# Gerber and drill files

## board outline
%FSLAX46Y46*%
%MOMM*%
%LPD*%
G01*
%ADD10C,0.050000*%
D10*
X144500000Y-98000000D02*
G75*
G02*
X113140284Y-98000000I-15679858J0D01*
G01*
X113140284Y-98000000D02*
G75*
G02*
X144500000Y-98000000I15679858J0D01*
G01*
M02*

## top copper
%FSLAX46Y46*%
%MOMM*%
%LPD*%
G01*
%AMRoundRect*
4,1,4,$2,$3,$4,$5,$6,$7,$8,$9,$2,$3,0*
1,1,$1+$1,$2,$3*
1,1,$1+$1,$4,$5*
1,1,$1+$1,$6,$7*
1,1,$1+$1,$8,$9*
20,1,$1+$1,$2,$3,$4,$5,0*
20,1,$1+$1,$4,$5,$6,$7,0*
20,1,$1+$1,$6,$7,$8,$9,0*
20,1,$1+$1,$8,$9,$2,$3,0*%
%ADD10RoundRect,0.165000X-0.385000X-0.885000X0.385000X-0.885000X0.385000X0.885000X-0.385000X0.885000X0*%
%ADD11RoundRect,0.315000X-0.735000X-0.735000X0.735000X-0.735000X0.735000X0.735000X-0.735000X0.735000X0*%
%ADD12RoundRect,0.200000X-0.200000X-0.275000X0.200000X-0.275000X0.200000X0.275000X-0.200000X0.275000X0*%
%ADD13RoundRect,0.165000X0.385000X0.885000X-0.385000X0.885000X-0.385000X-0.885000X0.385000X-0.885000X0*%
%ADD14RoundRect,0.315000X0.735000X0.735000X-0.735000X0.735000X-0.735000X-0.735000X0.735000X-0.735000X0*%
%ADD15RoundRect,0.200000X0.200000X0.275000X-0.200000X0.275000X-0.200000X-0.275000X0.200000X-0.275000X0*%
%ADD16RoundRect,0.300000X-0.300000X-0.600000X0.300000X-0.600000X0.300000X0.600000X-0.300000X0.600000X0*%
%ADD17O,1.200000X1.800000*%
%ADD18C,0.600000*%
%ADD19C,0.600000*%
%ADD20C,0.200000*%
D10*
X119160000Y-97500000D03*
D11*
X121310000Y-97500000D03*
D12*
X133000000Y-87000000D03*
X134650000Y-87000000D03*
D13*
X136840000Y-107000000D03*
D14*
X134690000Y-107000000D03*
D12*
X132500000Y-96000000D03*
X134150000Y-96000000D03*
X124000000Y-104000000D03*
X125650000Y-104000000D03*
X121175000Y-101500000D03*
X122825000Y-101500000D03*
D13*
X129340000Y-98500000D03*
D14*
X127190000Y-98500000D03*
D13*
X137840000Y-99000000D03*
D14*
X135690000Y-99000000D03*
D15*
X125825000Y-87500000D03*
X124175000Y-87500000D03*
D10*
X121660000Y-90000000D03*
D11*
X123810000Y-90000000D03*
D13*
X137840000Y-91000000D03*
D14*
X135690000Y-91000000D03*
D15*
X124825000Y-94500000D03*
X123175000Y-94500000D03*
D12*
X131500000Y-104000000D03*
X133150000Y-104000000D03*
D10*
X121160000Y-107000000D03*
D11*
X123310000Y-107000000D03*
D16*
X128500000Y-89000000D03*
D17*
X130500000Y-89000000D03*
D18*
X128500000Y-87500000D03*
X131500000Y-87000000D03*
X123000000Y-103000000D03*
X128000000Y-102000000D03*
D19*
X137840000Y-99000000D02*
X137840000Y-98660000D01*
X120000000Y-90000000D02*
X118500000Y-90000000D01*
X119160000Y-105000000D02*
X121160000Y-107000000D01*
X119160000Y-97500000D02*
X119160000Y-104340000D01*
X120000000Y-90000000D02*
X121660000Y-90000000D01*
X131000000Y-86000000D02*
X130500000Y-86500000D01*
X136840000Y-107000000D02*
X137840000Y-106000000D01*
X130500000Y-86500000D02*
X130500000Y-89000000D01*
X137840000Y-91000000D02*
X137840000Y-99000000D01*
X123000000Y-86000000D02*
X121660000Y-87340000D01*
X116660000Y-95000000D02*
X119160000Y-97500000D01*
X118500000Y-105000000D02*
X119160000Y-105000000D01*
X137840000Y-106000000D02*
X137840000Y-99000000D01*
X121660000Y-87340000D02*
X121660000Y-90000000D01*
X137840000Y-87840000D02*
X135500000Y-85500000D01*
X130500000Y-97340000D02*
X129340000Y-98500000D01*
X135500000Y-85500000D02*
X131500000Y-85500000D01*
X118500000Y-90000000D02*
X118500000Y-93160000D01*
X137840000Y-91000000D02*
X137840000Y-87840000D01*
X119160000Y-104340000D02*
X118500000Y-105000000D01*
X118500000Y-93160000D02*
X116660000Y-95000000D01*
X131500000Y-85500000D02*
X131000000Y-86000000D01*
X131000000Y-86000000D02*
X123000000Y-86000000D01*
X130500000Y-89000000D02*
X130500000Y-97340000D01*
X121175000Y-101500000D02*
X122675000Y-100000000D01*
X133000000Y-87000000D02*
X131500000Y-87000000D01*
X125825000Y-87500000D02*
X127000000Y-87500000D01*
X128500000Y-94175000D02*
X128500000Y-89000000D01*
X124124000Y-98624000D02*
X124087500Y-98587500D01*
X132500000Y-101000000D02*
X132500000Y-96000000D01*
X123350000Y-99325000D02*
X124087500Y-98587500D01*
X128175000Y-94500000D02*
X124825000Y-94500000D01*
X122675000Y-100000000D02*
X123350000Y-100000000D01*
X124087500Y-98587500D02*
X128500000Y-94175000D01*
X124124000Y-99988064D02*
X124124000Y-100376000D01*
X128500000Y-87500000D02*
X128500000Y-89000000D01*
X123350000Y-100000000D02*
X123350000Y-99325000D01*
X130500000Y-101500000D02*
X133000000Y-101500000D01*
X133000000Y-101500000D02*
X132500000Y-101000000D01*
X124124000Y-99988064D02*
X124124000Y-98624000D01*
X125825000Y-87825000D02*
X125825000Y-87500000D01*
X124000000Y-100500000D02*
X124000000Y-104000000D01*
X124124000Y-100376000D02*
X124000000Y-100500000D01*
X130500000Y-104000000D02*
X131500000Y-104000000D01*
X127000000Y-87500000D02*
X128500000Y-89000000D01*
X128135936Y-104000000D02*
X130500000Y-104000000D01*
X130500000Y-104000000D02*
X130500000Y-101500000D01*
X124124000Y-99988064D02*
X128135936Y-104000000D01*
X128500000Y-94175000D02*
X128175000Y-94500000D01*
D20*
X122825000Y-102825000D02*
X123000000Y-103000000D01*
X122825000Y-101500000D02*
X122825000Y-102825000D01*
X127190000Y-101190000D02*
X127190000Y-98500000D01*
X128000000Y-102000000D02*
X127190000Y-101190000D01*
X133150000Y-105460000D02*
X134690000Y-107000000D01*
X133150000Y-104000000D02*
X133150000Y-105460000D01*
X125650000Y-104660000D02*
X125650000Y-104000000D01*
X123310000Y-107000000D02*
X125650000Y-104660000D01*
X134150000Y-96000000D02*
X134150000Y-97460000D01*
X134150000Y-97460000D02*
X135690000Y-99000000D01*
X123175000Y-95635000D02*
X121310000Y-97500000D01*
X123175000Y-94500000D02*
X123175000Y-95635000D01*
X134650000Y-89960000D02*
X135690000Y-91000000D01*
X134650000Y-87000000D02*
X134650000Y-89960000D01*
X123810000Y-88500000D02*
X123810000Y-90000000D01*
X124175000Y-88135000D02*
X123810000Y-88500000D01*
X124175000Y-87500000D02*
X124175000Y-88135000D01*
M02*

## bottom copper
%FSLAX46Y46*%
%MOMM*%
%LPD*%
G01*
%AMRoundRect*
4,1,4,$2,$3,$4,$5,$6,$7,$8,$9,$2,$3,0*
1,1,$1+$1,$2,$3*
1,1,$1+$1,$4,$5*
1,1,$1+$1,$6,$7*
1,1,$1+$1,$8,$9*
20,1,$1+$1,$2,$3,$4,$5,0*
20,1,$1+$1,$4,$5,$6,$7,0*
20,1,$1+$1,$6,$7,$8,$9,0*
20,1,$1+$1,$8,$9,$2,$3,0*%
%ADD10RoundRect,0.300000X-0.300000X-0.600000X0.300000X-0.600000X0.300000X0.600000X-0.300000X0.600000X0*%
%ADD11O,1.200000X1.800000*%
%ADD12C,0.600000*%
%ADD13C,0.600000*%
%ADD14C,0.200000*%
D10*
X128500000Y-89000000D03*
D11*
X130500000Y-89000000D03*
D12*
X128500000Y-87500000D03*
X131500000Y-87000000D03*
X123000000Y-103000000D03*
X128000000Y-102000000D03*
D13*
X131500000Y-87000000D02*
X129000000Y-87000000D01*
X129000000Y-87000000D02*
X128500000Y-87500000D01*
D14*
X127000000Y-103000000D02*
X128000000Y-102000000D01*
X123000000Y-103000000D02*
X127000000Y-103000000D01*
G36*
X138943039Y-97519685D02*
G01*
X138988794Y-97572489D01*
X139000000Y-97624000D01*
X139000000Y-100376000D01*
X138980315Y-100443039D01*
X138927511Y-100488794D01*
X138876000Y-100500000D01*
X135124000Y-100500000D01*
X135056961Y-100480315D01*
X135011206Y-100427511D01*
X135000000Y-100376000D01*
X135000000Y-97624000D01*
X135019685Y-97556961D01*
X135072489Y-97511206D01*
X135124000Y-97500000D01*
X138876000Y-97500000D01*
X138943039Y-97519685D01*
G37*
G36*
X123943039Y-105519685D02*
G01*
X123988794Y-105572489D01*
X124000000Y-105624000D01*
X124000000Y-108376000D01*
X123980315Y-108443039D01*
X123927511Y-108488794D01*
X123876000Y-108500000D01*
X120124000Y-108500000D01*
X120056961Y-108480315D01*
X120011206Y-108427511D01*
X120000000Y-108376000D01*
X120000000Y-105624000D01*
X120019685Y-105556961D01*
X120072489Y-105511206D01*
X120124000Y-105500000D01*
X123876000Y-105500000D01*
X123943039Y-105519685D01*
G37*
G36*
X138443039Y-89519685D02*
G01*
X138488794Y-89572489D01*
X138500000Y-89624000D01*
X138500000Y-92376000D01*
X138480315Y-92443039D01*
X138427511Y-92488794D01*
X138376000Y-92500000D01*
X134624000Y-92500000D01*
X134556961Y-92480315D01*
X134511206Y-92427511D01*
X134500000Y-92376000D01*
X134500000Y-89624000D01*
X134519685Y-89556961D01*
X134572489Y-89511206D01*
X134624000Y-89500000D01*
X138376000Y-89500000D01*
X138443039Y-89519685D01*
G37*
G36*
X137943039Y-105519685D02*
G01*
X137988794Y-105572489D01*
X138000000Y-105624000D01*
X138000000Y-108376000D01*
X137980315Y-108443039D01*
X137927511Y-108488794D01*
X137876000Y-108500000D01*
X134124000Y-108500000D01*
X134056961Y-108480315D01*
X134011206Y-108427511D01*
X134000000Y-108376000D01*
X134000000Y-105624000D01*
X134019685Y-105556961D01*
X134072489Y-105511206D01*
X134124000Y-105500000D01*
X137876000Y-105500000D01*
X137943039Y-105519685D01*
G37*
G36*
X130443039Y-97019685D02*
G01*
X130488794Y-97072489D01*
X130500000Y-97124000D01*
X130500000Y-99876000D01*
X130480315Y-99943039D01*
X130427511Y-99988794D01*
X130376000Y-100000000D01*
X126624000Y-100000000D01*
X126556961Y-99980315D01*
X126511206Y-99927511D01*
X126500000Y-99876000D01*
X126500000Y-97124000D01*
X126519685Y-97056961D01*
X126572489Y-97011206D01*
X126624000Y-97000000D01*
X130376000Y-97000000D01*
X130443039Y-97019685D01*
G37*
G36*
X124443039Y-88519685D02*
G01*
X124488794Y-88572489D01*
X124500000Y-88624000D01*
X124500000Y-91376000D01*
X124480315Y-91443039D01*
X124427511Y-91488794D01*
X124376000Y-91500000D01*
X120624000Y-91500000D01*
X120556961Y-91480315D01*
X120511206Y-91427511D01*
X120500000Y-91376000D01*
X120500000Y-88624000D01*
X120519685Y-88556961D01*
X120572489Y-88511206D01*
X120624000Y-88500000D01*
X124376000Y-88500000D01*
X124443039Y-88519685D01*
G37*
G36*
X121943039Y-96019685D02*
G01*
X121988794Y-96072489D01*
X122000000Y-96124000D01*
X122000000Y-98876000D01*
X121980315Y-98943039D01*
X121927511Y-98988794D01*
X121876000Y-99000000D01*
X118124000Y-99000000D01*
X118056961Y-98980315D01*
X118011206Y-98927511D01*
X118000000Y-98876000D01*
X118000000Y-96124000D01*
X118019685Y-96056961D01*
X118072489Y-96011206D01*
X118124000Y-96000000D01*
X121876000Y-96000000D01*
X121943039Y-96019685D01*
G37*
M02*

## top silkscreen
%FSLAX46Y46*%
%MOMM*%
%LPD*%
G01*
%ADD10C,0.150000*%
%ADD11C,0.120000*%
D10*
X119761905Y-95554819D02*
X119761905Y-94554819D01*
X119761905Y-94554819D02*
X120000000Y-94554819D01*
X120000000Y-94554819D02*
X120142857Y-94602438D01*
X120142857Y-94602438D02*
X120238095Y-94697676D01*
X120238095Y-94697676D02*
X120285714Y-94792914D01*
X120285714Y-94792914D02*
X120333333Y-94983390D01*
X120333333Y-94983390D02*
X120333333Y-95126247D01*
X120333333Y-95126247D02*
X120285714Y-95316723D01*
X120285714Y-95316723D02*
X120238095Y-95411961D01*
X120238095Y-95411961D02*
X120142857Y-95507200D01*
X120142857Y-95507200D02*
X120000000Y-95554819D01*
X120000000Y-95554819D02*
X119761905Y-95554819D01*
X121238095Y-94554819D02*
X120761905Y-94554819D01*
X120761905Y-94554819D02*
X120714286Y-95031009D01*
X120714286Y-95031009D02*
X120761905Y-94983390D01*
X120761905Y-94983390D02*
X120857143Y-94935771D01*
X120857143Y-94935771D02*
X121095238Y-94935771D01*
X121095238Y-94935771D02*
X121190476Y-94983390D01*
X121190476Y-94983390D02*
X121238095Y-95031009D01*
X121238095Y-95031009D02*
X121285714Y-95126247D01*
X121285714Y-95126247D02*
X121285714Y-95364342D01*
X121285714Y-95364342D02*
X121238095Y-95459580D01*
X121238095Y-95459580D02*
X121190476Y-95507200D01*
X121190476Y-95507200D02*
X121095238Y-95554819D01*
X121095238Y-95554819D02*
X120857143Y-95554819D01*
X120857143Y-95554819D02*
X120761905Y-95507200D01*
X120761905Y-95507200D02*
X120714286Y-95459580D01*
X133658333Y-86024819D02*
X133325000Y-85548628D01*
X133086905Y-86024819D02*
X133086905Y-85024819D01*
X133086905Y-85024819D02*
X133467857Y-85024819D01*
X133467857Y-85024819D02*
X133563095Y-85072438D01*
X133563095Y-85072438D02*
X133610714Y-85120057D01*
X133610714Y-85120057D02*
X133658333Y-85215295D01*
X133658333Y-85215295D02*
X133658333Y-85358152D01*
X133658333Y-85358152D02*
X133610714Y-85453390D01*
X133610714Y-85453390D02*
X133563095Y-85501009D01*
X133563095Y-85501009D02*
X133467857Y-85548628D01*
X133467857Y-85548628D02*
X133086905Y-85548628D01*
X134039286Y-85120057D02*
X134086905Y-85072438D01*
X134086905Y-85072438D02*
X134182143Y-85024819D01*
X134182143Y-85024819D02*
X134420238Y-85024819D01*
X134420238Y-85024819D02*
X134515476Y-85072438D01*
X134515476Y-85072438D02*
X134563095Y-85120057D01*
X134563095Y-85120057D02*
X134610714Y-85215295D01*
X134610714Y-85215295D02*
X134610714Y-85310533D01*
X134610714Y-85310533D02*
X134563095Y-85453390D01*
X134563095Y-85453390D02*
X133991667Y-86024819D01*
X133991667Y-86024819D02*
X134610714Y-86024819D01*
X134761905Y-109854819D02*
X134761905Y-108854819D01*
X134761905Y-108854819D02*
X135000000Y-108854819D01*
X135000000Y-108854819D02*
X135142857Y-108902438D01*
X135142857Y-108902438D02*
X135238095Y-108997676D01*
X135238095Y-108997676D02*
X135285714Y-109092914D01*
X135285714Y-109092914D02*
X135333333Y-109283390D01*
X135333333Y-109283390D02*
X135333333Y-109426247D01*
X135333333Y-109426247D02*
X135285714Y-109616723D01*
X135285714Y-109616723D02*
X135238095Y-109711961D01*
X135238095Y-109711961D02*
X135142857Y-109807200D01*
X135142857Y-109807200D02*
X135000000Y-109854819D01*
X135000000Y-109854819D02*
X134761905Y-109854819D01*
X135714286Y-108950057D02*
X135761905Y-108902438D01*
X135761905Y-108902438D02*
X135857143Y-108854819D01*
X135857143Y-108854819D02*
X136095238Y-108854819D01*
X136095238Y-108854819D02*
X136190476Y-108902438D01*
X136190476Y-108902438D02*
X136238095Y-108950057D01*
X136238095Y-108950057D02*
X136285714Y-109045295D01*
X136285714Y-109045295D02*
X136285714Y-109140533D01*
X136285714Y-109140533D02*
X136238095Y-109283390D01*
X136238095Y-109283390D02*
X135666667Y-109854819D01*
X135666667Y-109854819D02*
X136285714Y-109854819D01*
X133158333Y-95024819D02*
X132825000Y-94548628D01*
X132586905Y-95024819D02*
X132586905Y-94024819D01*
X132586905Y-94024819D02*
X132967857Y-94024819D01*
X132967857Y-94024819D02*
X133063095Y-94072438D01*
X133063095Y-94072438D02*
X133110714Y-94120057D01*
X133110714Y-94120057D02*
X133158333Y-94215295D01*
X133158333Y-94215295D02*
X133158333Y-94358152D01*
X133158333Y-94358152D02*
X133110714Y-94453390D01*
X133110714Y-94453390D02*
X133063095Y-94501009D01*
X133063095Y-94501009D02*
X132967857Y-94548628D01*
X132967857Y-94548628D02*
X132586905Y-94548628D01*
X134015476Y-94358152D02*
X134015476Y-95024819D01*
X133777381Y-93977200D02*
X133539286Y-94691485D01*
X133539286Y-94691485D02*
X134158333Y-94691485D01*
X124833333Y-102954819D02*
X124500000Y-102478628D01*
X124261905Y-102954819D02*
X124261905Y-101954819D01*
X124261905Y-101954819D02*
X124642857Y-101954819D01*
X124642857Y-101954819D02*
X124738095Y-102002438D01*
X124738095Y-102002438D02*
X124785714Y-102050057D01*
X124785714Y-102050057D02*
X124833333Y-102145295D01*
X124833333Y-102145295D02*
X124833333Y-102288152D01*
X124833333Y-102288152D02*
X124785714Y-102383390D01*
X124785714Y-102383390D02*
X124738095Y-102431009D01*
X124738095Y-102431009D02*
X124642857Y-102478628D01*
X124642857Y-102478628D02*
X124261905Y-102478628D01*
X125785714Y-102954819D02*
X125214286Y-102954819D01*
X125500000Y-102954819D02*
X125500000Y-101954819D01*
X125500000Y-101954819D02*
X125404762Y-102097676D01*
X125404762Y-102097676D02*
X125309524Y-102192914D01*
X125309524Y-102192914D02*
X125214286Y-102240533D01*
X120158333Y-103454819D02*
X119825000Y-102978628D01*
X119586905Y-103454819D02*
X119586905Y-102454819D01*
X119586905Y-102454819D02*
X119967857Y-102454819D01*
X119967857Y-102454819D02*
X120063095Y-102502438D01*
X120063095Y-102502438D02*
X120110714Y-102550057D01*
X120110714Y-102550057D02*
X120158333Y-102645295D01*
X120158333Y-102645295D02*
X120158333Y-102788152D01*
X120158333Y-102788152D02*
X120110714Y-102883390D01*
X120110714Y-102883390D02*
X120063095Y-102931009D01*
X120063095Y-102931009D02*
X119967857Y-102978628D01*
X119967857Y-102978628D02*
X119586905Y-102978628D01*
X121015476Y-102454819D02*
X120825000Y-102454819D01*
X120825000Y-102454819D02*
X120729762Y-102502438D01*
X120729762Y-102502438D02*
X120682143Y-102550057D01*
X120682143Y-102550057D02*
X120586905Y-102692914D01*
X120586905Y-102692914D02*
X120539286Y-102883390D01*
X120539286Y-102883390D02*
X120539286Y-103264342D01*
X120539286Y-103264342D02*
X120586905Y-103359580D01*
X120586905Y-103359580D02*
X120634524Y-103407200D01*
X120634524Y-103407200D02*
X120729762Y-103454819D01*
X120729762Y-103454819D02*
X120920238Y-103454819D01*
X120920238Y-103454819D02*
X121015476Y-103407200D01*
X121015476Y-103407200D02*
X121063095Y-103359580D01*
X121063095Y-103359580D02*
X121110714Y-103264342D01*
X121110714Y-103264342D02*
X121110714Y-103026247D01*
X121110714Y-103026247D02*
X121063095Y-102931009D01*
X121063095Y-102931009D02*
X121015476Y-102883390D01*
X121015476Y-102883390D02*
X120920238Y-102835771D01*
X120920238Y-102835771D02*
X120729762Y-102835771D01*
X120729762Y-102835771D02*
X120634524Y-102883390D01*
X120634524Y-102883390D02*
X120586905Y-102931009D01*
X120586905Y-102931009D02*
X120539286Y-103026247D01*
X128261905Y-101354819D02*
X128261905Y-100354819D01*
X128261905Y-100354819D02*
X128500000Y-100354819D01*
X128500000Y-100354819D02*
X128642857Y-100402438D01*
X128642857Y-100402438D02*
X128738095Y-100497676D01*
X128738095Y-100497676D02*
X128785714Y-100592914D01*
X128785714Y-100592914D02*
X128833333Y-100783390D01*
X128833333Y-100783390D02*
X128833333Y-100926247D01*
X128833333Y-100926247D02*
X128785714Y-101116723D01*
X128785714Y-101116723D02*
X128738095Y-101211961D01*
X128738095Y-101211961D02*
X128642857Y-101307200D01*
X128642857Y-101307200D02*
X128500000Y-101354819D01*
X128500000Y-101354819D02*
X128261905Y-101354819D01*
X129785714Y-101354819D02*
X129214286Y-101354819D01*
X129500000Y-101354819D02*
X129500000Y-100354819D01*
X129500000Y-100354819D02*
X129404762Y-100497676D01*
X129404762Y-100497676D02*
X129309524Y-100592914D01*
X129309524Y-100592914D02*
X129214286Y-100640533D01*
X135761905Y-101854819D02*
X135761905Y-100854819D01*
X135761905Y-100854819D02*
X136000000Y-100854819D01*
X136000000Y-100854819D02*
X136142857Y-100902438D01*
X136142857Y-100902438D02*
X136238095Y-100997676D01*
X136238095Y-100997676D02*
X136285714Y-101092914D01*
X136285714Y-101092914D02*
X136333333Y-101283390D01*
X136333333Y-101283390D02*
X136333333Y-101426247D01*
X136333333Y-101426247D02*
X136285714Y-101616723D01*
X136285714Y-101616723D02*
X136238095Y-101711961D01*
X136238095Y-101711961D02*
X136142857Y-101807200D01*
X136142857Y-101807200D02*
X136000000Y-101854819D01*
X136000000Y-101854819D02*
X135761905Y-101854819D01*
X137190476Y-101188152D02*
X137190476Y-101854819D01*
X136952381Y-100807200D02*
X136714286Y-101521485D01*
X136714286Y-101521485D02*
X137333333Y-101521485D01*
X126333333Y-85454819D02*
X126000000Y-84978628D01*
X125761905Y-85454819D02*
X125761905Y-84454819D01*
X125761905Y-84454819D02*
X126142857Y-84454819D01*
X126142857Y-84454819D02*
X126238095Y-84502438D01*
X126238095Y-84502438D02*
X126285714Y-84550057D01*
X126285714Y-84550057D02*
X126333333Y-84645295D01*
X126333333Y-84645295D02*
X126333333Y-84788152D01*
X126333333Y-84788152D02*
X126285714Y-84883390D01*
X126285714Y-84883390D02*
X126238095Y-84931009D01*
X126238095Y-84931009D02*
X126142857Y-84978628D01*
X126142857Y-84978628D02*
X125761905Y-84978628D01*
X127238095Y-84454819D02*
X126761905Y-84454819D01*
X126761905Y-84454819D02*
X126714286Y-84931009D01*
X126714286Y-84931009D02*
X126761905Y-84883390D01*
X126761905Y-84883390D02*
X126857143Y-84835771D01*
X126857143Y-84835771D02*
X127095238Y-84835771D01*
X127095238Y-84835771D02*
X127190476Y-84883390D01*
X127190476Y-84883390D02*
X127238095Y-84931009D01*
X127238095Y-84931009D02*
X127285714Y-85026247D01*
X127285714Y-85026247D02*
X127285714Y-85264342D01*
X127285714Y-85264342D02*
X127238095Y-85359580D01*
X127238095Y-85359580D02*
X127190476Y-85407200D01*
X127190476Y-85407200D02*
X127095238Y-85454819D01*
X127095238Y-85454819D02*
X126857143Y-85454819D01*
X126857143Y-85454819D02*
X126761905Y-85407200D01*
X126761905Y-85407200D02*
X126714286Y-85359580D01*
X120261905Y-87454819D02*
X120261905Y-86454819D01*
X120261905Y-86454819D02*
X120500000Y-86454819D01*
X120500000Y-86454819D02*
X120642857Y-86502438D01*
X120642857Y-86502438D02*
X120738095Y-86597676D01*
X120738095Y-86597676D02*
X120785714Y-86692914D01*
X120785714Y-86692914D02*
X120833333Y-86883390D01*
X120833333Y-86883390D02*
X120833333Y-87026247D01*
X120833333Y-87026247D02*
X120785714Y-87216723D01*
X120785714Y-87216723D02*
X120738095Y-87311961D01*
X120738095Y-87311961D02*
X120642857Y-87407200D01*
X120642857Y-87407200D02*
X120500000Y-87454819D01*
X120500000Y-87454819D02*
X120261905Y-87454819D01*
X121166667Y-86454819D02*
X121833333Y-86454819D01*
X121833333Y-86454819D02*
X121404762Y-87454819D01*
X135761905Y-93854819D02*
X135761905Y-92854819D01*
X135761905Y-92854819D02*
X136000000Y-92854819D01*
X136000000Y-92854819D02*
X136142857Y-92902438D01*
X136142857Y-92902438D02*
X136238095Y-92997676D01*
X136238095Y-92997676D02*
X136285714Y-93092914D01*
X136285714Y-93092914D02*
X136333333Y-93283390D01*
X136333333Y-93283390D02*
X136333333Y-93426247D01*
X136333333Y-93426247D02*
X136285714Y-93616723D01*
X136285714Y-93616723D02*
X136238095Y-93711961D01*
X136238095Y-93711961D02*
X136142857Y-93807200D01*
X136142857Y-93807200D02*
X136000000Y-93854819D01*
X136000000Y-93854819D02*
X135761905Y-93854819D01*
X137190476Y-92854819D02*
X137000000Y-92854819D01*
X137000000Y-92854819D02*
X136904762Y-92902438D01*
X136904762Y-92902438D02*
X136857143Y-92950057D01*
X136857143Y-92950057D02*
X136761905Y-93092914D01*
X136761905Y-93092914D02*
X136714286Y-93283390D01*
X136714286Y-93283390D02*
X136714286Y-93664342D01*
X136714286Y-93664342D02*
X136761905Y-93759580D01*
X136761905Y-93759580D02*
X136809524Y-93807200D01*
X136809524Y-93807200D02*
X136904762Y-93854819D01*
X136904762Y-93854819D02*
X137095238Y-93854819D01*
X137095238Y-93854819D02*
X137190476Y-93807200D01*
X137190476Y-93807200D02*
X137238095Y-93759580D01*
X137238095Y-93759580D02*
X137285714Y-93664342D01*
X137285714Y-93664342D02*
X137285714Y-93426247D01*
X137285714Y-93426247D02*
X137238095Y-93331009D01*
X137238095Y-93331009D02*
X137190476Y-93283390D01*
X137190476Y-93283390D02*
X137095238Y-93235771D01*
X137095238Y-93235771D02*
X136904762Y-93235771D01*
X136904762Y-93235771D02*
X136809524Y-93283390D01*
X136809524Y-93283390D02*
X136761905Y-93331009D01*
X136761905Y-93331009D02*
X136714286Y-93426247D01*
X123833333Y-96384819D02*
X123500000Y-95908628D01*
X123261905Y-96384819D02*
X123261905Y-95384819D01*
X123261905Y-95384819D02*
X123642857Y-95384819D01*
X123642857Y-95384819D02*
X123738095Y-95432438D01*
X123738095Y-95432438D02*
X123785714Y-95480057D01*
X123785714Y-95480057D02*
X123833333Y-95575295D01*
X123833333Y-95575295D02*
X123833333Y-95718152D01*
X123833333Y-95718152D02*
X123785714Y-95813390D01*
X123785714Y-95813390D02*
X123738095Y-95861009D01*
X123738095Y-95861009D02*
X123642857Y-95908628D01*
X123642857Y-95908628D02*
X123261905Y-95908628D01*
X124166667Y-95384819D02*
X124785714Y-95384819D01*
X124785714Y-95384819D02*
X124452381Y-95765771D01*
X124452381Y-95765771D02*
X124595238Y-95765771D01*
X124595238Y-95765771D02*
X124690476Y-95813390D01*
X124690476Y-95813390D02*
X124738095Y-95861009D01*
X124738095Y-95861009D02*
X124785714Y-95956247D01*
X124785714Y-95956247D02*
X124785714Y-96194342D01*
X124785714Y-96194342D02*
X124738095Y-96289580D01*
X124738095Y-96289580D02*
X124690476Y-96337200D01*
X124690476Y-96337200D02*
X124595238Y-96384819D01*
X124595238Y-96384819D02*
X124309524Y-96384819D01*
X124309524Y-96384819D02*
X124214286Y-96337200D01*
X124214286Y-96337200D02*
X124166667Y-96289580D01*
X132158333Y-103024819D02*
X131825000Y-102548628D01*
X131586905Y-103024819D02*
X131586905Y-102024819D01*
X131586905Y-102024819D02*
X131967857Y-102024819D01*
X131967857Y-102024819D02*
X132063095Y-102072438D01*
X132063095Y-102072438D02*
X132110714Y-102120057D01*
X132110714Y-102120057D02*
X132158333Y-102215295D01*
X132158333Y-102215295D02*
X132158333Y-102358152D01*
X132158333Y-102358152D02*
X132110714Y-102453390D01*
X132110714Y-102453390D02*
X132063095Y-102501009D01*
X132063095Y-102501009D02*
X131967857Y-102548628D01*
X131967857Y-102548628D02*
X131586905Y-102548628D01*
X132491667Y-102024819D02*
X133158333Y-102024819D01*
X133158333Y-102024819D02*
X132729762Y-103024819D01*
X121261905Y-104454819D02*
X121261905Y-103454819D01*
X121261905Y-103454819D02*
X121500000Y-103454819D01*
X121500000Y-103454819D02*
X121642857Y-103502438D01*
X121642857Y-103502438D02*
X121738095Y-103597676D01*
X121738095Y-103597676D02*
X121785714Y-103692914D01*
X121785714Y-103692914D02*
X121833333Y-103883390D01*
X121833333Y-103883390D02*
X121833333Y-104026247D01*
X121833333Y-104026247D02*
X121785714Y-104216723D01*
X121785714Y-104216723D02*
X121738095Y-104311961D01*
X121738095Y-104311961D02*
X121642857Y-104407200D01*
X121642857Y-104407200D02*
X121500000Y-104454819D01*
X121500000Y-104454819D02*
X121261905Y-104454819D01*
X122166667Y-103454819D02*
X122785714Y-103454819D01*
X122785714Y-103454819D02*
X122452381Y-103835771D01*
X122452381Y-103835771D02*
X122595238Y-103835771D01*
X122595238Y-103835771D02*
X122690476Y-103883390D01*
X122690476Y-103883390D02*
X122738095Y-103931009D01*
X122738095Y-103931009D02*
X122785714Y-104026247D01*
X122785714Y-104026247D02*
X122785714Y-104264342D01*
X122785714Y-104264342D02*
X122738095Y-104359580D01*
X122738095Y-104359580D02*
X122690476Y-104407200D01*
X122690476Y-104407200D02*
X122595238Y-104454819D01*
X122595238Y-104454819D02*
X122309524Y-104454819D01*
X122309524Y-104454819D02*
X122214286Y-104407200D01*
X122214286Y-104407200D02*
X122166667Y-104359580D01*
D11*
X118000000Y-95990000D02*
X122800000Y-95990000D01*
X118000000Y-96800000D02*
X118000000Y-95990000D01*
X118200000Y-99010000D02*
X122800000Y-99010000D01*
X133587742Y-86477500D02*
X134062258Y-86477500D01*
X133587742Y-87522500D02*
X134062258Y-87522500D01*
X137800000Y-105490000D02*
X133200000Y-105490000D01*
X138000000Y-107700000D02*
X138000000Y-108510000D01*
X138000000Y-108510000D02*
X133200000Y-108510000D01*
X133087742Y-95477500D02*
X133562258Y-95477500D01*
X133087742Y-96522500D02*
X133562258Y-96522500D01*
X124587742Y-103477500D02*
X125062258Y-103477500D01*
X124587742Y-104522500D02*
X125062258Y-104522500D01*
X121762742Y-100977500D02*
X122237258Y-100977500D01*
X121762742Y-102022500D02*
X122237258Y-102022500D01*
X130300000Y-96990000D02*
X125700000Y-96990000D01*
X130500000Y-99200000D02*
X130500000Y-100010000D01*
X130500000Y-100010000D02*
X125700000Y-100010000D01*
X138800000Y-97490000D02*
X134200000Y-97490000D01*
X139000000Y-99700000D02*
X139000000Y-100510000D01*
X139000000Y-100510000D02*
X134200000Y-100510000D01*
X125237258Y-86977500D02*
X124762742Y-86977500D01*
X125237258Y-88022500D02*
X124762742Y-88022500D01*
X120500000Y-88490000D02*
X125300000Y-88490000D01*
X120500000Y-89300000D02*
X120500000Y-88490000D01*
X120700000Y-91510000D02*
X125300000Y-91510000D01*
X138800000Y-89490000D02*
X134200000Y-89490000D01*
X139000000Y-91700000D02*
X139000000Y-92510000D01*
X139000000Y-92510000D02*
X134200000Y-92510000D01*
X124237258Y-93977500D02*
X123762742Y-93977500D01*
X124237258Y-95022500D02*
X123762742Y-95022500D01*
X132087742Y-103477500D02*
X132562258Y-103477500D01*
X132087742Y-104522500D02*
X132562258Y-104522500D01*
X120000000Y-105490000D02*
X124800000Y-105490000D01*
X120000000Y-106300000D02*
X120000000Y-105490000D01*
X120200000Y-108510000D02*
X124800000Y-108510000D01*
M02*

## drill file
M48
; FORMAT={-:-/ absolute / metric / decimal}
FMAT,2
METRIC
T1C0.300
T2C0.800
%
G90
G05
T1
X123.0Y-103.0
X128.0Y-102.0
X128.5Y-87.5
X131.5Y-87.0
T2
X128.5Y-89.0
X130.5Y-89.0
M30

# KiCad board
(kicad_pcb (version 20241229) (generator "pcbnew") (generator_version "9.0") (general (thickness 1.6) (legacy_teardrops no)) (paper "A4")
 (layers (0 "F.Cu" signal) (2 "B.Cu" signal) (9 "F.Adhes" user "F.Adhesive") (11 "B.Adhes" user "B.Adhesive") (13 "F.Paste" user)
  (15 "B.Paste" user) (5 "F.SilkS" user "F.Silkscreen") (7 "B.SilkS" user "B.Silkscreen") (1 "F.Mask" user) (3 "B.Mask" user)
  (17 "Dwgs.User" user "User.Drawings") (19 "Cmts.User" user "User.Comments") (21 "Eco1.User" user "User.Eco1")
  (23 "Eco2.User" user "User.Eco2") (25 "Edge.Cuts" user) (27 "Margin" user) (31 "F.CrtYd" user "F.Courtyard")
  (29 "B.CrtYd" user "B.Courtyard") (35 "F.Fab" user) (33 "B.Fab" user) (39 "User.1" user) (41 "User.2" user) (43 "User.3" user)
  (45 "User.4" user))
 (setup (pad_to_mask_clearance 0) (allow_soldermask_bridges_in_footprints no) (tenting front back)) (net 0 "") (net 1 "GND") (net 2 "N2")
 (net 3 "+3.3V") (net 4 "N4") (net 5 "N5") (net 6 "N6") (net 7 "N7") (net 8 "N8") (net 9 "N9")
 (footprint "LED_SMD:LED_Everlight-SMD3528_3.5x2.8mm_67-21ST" (layer "F.Cu") (at 120.5 97.5)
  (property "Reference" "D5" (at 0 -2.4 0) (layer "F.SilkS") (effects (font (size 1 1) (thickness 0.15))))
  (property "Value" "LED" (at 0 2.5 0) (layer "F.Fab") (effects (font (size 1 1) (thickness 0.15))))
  (fp_line (start -2.5 -1.51) (end 2.3 -1.51) (stroke (width 0.12) (type solid)) (layer "F.SilkS"))
  (fp_line (start -2.5 -0.7) (end -2.5 -1.51) (stroke (width 0.12) (type solid)) (layer "F.SilkS"))
  (fp_line (start -2.3 1.51) (end 2.3 1.51) (stroke (width 0.12) (type solid)) (layer "F.SilkS"))
  (pad "1" smd roundrect (at -1.34 0) (size 1.1 2.1) (layers "F.Cu" "F.Mask" "F.Paste") (roundrect_rratio 0.15) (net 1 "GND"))
  (pad "2" smd roundrect (at 0.81 0) (size 2.1 2.1) (layers "F.Cu" "F.Mask" "F.Paste") (roundrect_rratio 0.15) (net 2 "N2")))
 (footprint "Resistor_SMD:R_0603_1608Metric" (layer "F.Cu") (at 133.825 87)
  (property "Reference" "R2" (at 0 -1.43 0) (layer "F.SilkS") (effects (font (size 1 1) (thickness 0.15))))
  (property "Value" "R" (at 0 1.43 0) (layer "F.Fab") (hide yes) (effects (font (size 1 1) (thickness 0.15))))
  (fp_line (start -0.237258 -0.5225) (end 0.237258 -0.5225) (stroke (width 0.12) (type solid)) (layer "F.SilkS"))
  (fp_line (start -0.237258 0.5225) (end 0.237258 0.5225) (stroke (width 0.12) (type solid)) (layer "F.SilkS"))
  (pad "1" smd roundrect (at -0.825 0) (size 0.8 0.95) (layers "F.Cu" "F.Mask" "F.Paste") (roundrect_rratio 0.25) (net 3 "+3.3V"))
  (pad "2" smd roundrect (at 0.825 0) (size 0.8 0.95) (layers "F.Cu" "F.Mask" "F.Paste") (roundrect_rratio 0.25) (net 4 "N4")))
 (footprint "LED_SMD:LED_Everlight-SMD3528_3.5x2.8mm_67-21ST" (layer "F.Cu") (at 135.5 107 180)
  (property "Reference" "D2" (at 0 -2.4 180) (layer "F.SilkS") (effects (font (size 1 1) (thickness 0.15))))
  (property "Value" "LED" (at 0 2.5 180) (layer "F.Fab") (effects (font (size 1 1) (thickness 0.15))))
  (fp_line (start -2.3 1.51) (end 2.3 1.51) (stroke (width 0.12) (type solid)) (layer "F.SilkS"))
  (fp_line (start -2.5 -0.7) (end -2.5 -1.51) (stroke (width 0.12) (type solid)) (layer "F.SilkS"))
  (fp_line (start -2.5 -1.51) (end 2.3 -1.51) (stroke (width 0.12) (type solid)) (layer "F.SilkS"))
  (pad "1" smd roundrect (at -1.34 0 180) (size 1.1 2.1) (layers "F.Cu" "F.Mask" "F.Paste") (roundrect_rratio 0.15) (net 1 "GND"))
  (pad "2" smd roundrect (at 0.81 0 180) (size 2.1 2.1) (layers "F.Cu" "F.Mask" "F.Paste") (roundrect_rratio 0.15) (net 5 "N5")))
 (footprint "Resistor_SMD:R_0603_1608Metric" (layer "F.Cu") (at 133.325 96)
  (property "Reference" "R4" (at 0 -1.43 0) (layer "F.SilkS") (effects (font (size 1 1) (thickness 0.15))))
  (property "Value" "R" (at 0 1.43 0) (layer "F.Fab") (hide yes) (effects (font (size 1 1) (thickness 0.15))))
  (fp_line (start -0.237258 -0.5225) (end 0.237258 -0.5225) (stroke (width 0.12) (type solid)) (layer "F.SilkS"))
  (fp_line (start -0.237258 0.5225) (end 0.237258 0.5225) (stroke (width 0.12) (type solid)) (layer "F.SilkS"))
  (pad "1" smd roundrect (at -0.825 0) (size 0.8 0.95) (layers "F.Cu" "F.Mask" "F.Paste") (roundrect_rratio 0.25) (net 3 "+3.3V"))
  (pad "2" smd roundrect (at 0.825 0) (size 0.8 0.95) (layers "F.Cu" "F.Mask" "F.Paste") (roundrect_rratio 0.25) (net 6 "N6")))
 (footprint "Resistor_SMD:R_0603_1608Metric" (layer "F.Cu") (at 124.825 104)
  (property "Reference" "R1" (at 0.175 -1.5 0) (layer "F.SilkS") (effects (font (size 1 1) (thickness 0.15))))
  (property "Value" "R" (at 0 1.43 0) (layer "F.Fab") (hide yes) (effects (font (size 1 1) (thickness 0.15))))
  (fp_line (start -0.237258 -0.5225) (end 0.237258 -0.5225) (stroke (width 0.12) (type solid)) (layer "F.SilkS"))
  (fp_line (start -0.237258 0.5225) (end 0.237258 0.5225) (stroke (width 0.12) (type solid)) (layer "F.SilkS"))
  (pad "1" smd roundrect (at -0.825 0) (size 0.8 0.95) (layers "F.Cu" "F.Mask" "F.Paste") (roundrect_rratio 0.25) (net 3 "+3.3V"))
  (pad "2" smd roundrect (at 0.825 0) (size 0.8 0.95) (layers "F.Cu" "F.Mask" "F.Paste") (roundrect_rratio 0.25) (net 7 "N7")))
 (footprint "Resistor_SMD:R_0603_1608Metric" (layer "F.Cu") (at 122 101.5)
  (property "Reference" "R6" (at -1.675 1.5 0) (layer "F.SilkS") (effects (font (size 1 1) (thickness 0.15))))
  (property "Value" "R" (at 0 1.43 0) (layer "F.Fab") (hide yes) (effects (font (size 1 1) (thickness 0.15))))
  (fp_line (start -0.237258 -0.5225) (end 0.237258 -0.5225) (stroke (width 0.12) (type solid)) (layer "F.SilkS"))
  (fp_line (start -0.237258 0.5225) (end 0.237258 0.5225) (stroke (width 0.12) (type solid)) (layer "F.SilkS"))
  (pad "1" smd roundrect (at -0.825 0) (size 0.8 0.95) (layers "F.Cu" "F.Mask" "F.Paste") (roundrect_rratio 0.25) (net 3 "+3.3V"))
  (pad "2" smd roundrect (at 0.825 0) (size 0.8 0.95) (layers "F.Cu" "F.Mask" "F.Paste") (roundrect_rratio 0.25) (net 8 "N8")))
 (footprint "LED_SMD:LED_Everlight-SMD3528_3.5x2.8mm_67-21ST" (layer "F.Cu") (at 128 98.5 180)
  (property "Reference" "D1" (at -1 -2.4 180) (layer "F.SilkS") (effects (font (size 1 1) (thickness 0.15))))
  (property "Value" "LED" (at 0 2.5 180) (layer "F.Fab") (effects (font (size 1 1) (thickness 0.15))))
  (fp_line (start -2.3 1.51) (end 2.3 1.51) (stroke (width 0.12) (type solid)) (layer "F.SilkS"))
  (fp_line (start -2.5 -0.7) (end -2.5 -1.51) (stroke (width 0.12) (type solid)) (layer "F.SilkS"))
  (fp_line (start -2.5 -1.51) (end 2.3 -1.51) (stroke (width 0.12) (type solid)) (layer "F.SilkS"))
  (pad "1" smd roundrect (at -1.34 0 180) (size 1.1 2.1) (layers "F.Cu" "F.Mask" "F.Paste") (roundrect_rratio 0.15) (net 1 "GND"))
  (pad "2" smd roundrect (at 0.81 0 180) (size 2.1 2.1) (layers "F.Cu" "F.Mask" "F.Paste") (roundrect_rratio 0.15) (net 8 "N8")))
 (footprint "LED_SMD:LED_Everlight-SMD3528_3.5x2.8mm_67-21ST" (layer "F.Cu") (at 136.5 99 180)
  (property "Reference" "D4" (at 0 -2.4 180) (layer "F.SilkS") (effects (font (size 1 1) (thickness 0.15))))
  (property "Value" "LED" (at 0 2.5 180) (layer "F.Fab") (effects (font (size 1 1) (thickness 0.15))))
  (fp_line (start -2.3 1.51) (end 2.3 1.51) (stroke (width 0.12) (type solid)) (layer "F.SilkS"))
  (fp_line (start -2.5 -0.7) (end -2.5 -1.51) (stroke (width 0.12) (type solid)) (layer "F.SilkS"))
  (fp_line (start -2.5 -1.51) (end 2.3 -1.51) (stroke (width 0.12) (type solid)) (layer "F.SilkS"))
  (pad "1" smd roundrect (at -1.34 0 180) (size 1.1 2.1) (layers "F.Cu" "F.Mask" "F.Paste") (roundrect_rratio 0.15) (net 1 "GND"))
  (pad "2" smd roundrect (at 0.81 0 180) (size 2.1 2.1) (layers "F.Cu" "F.Mask" "F.Paste") (roundrect_rratio 0.15) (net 6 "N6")))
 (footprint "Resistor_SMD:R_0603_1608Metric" (layer "F.Cu") (at 125 87.5 180)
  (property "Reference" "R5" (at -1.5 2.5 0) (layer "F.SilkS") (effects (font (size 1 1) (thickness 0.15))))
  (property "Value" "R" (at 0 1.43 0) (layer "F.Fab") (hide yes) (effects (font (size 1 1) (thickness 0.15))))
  (fp_line (start -0.237258 0.5225) (end 0.237258 0.5225) (stroke (width 0.12) (type solid)) (layer "F.SilkS"))
  (fp_line (start -0.237258 -0.5225) (end 0.237258 -0.5225) (stroke (width 0.12) (type solid)) (layer "F.SilkS"))
  (pad "1" smd roundrect (at -0.825 0 180) (size 0.8 0.95) (layers "F.Cu" "F.Mask" "F.Paste") (roundrect_rratio 0.25) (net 3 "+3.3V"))
  (pad "2" smd roundrect (at 0.825 0 180) (size 0.8 0.95) (layers "F.Cu" "F.Mask" "F.Paste") (roundrect_rratio 0.25) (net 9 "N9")))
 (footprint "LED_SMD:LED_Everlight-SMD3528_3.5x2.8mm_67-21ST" (layer "F.Cu") (at 123 90)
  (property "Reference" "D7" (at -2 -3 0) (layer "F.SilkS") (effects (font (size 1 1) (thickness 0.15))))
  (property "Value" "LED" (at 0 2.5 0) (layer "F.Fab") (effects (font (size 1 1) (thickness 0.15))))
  (fp_line (start -2.5 -1.51) (end 2.3 -1.51) (stroke (width 0.12) (type solid)) (layer "F.SilkS"))
  (fp_line (start -2.5 -0.7) (end -2.5 -1.51) (stroke (width 0.12) (type solid)) (layer "F.SilkS"))
  (fp_line (start -2.3 1.51) (end 2.3 1.51) (stroke (width 0.12) (type solid)) (layer "F.SilkS"))
  (pad "1" smd roundrect (at -1.34 0) (size 1.1 2.1) (layers "F.Cu" "F.Mask" "F.Paste") (roundrect_rratio 0.15) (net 1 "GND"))
  (pad "2" smd roundrect (at 0.81 0) (size 2.1 2.1) (layers "F.Cu" "F.Mask" "F.Paste") (roundrect_rratio 0.15) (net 9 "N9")))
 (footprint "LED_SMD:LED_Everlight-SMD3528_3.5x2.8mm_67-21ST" (layer "F.Cu") (at 136.5 91 180)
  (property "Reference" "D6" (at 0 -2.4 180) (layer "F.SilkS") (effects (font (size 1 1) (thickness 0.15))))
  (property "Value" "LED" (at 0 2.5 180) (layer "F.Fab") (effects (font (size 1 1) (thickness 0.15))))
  (fp_line (start -2.3 1.51) (end 2.3 1.51) (stroke (width 0.12) (type solid)) (layer "F.SilkS"))
  (fp_line (start -2.5 -0.7) (end -2.5 -1.51) (stroke (width 0.12) (type solid)) (layer "F.SilkS"))
  (fp_line (start -2.5 -1.51) (end 2.3 -1.51) (stroke (width 0.12) (type solid)) (layer "F.SilkS"))
  (pad "1" smd roundrect (at -1.34 0 180) (size 1.1 2.1) (layers "F.Cu" "F.Mask" "F.Paste") (roundrect_rratio 0.15) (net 1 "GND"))
  (pad "2" smd roundrect (at 0.81 0 180) (size 2.1 2.1) (layers "F.Cu" "F.Mask" "F.Paste") (roundrect_rratio 0.15) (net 4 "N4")))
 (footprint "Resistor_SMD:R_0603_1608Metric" (layer "F.Cu") (at 124 94.5 180)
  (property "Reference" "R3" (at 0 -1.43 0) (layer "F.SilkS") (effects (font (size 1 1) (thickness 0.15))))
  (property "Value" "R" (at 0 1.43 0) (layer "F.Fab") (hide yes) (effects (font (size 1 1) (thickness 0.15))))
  (fp_line (start -0.237258 0.5225) (end 0.237258 0.5225) (stroke (width 0.12) (type solid)) (layer "F.SilkS"))
  (fp_line (start -0.237258 -0.5225) (end 0.237258 -0.5225) (stroke (width 0.12) (type solid)) (layer "F.SilkS"))
  (pad "1" smd roundrect (at -0.825 0 180) (size 0.8 0.95) (layers "F.Cu" "F.Mask" "F.Paste") (roundrect_rratio 0.25) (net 3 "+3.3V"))
  (pad "2" smd roundrect (at 0.825 0 180) (size 0.8 0.95) (layers "F.Cu" "F.Mask" "F.Paste") (roundrect_rratio 0.25) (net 2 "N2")))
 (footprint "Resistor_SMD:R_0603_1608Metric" (layer "F.Cu") (at 132.325 104)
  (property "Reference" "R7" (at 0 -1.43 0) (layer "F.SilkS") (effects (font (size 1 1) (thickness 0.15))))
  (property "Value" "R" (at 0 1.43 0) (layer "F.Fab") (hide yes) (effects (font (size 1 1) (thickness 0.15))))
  (fp_line (start -0.237258 -0.5225) (end 0.237258 -0.5225) (stroke (width 0.12) (type solid)) (layer "F.SilkS"))
  (fp_line (start -0.237258 0.5225) (end 0.237258 0.5225) (stroke (width 0.12) (type solid)) (layer "F.SilkS"))
  (pad "1" smd roundrect (at -0.825 0) (size 0.8 0.95) (layers "F.Cu" "F.Mask" "F.Paste") (roundrect_rratio 0.25) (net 3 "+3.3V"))
  (pad "2" smd roundrect (at 0.825 0) (size 0.8 0.95) (layers "F.Cu" "F.Mask" "F.Paste") (roundrect_rratio 0.25) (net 5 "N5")))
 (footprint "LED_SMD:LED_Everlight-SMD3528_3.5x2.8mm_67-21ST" (layer "F.Cu") (at 122.5 107)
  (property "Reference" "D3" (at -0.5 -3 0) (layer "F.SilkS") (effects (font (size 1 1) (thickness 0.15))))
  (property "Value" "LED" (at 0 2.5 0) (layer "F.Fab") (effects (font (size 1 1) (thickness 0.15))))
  (fp_line (start -2.5 -1.51) (end 2.3 -1.51) (stroke (width 0.12) (type solid)) (layer "F.SilkS"))
  (fp_line (start -2.5 -0.7) (end -2.5 -1.51) (stroke (width 0.12) (type solid)) (layer "F.SilkS"))
  (fp_line (start -2.3 1.51) (end 2.3 1.51) (stroke (width 0.12) (type solid)) (layer "F.SilkS"))
  (pad "1" smd roundrect (at -1.34 0) (size 1.1 2.1) (layers "F.Cu" "F.Mask" "F.Paste") (roundrect_rratio 0.15) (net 1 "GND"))
  (pad "2" smd roundrect (at 0.81 0) (size 2.1 2.1) (layers "F.Cu" "F.Mask" "F.Paste") (roundrect_rratio 0.15) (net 7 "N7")))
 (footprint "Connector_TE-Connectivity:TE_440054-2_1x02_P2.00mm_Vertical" (layer "B.Cu") (at 128.5 89)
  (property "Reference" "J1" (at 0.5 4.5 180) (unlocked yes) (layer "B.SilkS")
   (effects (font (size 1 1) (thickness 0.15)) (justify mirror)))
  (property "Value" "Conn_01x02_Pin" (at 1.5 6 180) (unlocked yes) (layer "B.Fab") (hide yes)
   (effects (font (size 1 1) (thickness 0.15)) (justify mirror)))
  (pad "1" thru_hole roundrect (at 0 0) (size 1.2 1.8) (drill 0.8) (layers "*.Cu" "*.Mask") (remove_unused_layers no)
   (roundrect_rratio 0.25) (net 3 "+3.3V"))
  (pad "2" thru_hole oval (at 2 0) (size 1.2 1.8) (drill 0.8) (layers "*.Cu" "*.Mask") (remove_unused_layers no) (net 1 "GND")))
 (gr_circle (center 128.820142 98) (end 130.320142 82.392055) (stroke (width 0.05) (type default)) (fill no) (layer "Edge.Cuts"))
 (segment (start 137.84 99) (end 137.84 98.66) (width 0.6) (layer "F.Cu") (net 1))
 (segment (start 120 90) (end 118.5 90) (width 0.6) (layer "F.Cu") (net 1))
 (segment (start 119.16 105) (end 121.16 107) (width 0.6) (layer "F.Cu") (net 1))
 (segment (start 119.16 97.5) (end 119.16 104.34) (width 0.6) (layer "F.Cu") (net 1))
 (segment (start 120 90) (end 121.66 90) (width 0.6) (layer "F.Cu") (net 1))
 (segment (start 131 86) (end 130.5 86.5) (width 0.6) (layer "F.Cu") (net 1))
 (segment (start 136.84 107) (end 137.84 106) (width 0.6) (layer "F.Cu") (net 1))
 (segment (start 130.5 86.5) (end 130.5 89) (width 0.6) (layer "F.Cu") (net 1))
 (segment (start 137.84 91) (end 137.84 99) (width 0.6) (layer "F.Cu") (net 1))
 (segment (start 123 86) (end 121.66 87.34) (width 0.6) (layer "F.Cu") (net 1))
 (segment (start 116.66 95) (end 119.16 97.5) (width 0.6) (layer "F.Cu") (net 1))
 (segment (start 118.5 105) (end 119.16 105) (width 0.6) (layer "F.Cu") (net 1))
 (segment (start 137.84 106) (end 137.84 99) (width 0.6) (layer "F.Cu") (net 1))
 (segment (start 121.66 87.34) (end 121.66 90) (width 0.6) (layer "F.Cu") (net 1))
 (segment (start 137.84 87.84) (end 135.5 85.5) (width 0.6) (layer "F.Cu") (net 1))
 (segment (start 130.5 97.34) (end 129.34 98.5) (width 0.6) (layer "F.Cu") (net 1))
 (segment (start 135.5 85.5) (end 131.5 85.5) (width 0.6) (layer "F.Cu") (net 1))
 (segment (start 118.5 90) (end 118.5 93.16) (width 0.6) (layer "F.Cu") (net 1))
 (segment (start 137.84 91) (end 137.84 87.84) (width 0.6) (layer "F.Cu") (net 1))
 (segment (start 119.16 104.34) (end 118.5 105) (width 0.6) (layer "F.Cu") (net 1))
 (segment (start 118.5 93.16) (end 116.66 95) (width 0.6) (layer "F.Cu") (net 1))
 (segment (start 131.5 85.5) (end 131 86) (width 0.6) (layer "F.Cu") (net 1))
 (segment (start 131 86) (end 123 86) (width 0.6) (layer "F.Cu") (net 1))
 (segment (start 130.5 89) (end 130.5 97.34) (width 0.6) (layer "F.Cu") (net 1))
 (segment (start 121.175 101.5) (end 122.675 100) (width 0.6) (layer "F.Cu") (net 3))
 (segment (start 133 87) (end 131.5 87) (width 0.6) (layer "F.Cu") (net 3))
 (segment (start 125.825 87.5) (end 127 87.5) (width 0.6) (layer "F.Cu") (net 3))
 (segment (start 128.5 94.175) (end 128.5 89) (width 0.6) (layer "F.Cu") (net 3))
 (segment (start 124.124 98.624) (end 124.0875 98.5875) (width 0.6) (layer "F.Cu") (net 3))
 (segment (start 132.5 101) (end 132.5 96) (width 0.6) (layer "F.Cu") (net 3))
 (segment (start 123.35 99.325) (end 124.0875 98.5875) (width 0.6) (layer "F.Cu") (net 3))
 (segment (start 128.175 94.5) (end 124.825 94.5) (width 0.6) (layer "F.Cu") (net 3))
 (segment (start 122.675 100) (end 123.35 100) (width 0.6) (layer "F.Cu") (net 3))
 (segment (start 124.0875 98.5875) (end 128.5 94.175) (width 0.6) (layer "F.Cu") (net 3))
 (segment (start 124.124 99.988064) (end 124.124 100.376) (width 0.6) (layer "F.Cu") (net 3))
 (segment (start 128.5 87.5) (end 128.5 89) (width 0.6) (layer "F.Cu") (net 3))
 (segment (start 123.35 100) (end 123.35 99.325) (width 0.6) (layer "F.Cu") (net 3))
 (segment (start 130.5 101.5) (end 133 101.5) (width 0.6) (layer "F.Cu") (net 3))
 (segment (start 133 101.5) (end 132.5 101) (width 0.6) (layer "F.Cu") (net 3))
 (segment (start 124.124 99.988064) (end 124.124 98.624) (width 0.6) (layer "F.Cu") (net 3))
 (segment (start 125.825 87.825) (end 125.825 87.5) (width 0.6) (layer "F.Cu") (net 3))
 (segment (start 124 100.5) (end 124 104) (width 0.6) (layer "F.Cu") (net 3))
 (segment (start 124.124 100.376) (end 124 100.5) (width 0.6) (layer "F.Cu") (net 3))
 (segment (start 130.5 104) (end 131.5 104) (width 0.6) (layer "F.Cu") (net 3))
 (segment (start 127 87.5) (end 128.5 89) (width 0.6) (layer "F.Cu") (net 3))
 (segment (start 128.135936 104) (end 130.5 104) (width 0.6) (layer "F.Cu") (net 3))
 (segment (start 130.5 104) (end 130.5 101.5) (width 0.6) (layer "F.Cu") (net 3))
 (segment (start 124.124 99.988064) (end 128.135936 104) (width 0.6) (layer "F.Cu") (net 3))
 (segment (start 128.5 94.175) (end 128.175 94.5) (width 0.6) (layer "F.Cu") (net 3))
 (via (at 128.5 87.5) (size 0.6) (drill 0.3) (layers "F.Cu" "B.Cu") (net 3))
 (via (at 131.5 87) (size 0.6) (drill 0.3) (layers "F.Cu" "B.Cu") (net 3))
 (segment (start 131.5 87) (end 129 87) (width 0.6) (layer "B.Cu") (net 3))
 (segment (start 129 87) (end 128.5 87.5) (width 0.6) (layer "B.Cu") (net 3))
 (segment (start 122.825 102.825) (end 123 103) (width 0.2) (layer "F.Cu") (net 8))
 (segment (start 122.825 101.5) (end 122.825 102.825) (width 0.2) (layer "F.Cu") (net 8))
 (segment (start 127.19 101.19) (end 127.19 98.5) (width 0.2) (layer "F.Cu") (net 8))
 (segment (start 128 102) (end 127.19 101.19) (width 0.2) (layer "F.Cu") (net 8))
 (via (at 123 103) (size 0.6) (drill 0.3) (layers "F.Cu" "B.Cu") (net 8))
 (via (at 128 102) (size 0.6) (drill 0.3) (layers "F.Cu" "B.Cu") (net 8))
 (segment (start 127 103) (end 128 102) (width 0.2) (layer "B.Cu") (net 8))
 (segment (start 123 103) (end 127 103) (width 0.2) (layer "B.Cu") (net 8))
 (segment (start 133.15 105.46) (end 134.69 107) (width 0.2) (layer "F.Cu") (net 5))
 (segment (start 133.15 104) (end 133.15 105.46) (width 0.2) (layer "F.Cu") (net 5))
 (segment (start 125.65 104.66) (end 125.65 104) (width 0.2) (layer "F.Cu") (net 7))
 (segment (start 123.31 107) (end 125.65 104.66) (width 0.2) (layer "F.Cu") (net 7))
 (segment (start 134.15 96) (end 134.15 97.46) (width 0.2) (layer "F.Cu") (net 6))
 (segment (start 134.15 97.46) (end 135.69 99) (width 0.2) (layer "F.Cu") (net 6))
 (segment (start 123.175 95.635) (end 121.31 97.5) (width 0.2) (layer "F.Cu") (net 2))
 (segment (start 123.175 94.5) (end 123.175 95.635) (width 0.2) (layer "F.Cu") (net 2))
 (segment (start 134.65 89.96) (end 135.69 91) (width 0.2) (layer "F.Cu") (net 4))
 (segment (start 134.65 87) (end 134.65 89.96) (width 0.2) (layer "F.Cu") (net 4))
 (segment (start 123.81 88.5) (end 123.81 90) (width 0.2) (layer "F.Cu") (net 9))
 (segment (start 124.175 88.135) (end 123.81 88.5) (width 0.2) (layer "F.Cu") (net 9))
 (segment (start 124.175 87.5) (end 124.175 88.135) (width 0.2) (layer "F.Cu") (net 9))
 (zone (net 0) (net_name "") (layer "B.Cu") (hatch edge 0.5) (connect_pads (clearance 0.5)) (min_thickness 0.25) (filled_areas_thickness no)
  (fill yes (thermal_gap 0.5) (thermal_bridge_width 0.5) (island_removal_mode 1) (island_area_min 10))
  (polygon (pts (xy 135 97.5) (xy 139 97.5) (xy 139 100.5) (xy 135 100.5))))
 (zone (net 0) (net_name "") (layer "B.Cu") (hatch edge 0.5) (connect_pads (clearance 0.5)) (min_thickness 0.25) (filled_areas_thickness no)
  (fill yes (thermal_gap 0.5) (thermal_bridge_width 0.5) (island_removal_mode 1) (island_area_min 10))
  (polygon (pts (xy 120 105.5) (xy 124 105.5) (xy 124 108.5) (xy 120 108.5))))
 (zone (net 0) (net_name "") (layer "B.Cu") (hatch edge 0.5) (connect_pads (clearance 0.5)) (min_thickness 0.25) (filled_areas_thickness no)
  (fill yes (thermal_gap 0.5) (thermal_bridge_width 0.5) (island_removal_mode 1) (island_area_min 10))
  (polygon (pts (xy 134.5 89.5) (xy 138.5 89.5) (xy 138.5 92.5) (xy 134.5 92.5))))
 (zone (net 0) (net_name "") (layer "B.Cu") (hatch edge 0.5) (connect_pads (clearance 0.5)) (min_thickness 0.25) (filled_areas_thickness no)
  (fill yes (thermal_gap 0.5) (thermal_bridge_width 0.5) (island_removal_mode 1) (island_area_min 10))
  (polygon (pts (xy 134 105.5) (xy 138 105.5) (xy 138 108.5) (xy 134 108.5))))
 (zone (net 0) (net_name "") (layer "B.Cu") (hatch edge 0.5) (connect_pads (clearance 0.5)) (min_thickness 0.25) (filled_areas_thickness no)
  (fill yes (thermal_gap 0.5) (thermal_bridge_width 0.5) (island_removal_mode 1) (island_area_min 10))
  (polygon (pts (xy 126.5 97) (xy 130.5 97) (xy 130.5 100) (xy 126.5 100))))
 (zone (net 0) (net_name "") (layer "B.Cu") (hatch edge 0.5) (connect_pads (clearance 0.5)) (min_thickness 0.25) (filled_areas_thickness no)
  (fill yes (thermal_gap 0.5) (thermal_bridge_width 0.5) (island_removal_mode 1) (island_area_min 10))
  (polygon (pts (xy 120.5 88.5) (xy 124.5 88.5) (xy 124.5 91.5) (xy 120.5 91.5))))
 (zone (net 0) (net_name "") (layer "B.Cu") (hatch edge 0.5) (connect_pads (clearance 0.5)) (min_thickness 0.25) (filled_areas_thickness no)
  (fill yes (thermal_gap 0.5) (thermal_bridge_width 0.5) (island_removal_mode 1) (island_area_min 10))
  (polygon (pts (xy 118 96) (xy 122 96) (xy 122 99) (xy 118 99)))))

